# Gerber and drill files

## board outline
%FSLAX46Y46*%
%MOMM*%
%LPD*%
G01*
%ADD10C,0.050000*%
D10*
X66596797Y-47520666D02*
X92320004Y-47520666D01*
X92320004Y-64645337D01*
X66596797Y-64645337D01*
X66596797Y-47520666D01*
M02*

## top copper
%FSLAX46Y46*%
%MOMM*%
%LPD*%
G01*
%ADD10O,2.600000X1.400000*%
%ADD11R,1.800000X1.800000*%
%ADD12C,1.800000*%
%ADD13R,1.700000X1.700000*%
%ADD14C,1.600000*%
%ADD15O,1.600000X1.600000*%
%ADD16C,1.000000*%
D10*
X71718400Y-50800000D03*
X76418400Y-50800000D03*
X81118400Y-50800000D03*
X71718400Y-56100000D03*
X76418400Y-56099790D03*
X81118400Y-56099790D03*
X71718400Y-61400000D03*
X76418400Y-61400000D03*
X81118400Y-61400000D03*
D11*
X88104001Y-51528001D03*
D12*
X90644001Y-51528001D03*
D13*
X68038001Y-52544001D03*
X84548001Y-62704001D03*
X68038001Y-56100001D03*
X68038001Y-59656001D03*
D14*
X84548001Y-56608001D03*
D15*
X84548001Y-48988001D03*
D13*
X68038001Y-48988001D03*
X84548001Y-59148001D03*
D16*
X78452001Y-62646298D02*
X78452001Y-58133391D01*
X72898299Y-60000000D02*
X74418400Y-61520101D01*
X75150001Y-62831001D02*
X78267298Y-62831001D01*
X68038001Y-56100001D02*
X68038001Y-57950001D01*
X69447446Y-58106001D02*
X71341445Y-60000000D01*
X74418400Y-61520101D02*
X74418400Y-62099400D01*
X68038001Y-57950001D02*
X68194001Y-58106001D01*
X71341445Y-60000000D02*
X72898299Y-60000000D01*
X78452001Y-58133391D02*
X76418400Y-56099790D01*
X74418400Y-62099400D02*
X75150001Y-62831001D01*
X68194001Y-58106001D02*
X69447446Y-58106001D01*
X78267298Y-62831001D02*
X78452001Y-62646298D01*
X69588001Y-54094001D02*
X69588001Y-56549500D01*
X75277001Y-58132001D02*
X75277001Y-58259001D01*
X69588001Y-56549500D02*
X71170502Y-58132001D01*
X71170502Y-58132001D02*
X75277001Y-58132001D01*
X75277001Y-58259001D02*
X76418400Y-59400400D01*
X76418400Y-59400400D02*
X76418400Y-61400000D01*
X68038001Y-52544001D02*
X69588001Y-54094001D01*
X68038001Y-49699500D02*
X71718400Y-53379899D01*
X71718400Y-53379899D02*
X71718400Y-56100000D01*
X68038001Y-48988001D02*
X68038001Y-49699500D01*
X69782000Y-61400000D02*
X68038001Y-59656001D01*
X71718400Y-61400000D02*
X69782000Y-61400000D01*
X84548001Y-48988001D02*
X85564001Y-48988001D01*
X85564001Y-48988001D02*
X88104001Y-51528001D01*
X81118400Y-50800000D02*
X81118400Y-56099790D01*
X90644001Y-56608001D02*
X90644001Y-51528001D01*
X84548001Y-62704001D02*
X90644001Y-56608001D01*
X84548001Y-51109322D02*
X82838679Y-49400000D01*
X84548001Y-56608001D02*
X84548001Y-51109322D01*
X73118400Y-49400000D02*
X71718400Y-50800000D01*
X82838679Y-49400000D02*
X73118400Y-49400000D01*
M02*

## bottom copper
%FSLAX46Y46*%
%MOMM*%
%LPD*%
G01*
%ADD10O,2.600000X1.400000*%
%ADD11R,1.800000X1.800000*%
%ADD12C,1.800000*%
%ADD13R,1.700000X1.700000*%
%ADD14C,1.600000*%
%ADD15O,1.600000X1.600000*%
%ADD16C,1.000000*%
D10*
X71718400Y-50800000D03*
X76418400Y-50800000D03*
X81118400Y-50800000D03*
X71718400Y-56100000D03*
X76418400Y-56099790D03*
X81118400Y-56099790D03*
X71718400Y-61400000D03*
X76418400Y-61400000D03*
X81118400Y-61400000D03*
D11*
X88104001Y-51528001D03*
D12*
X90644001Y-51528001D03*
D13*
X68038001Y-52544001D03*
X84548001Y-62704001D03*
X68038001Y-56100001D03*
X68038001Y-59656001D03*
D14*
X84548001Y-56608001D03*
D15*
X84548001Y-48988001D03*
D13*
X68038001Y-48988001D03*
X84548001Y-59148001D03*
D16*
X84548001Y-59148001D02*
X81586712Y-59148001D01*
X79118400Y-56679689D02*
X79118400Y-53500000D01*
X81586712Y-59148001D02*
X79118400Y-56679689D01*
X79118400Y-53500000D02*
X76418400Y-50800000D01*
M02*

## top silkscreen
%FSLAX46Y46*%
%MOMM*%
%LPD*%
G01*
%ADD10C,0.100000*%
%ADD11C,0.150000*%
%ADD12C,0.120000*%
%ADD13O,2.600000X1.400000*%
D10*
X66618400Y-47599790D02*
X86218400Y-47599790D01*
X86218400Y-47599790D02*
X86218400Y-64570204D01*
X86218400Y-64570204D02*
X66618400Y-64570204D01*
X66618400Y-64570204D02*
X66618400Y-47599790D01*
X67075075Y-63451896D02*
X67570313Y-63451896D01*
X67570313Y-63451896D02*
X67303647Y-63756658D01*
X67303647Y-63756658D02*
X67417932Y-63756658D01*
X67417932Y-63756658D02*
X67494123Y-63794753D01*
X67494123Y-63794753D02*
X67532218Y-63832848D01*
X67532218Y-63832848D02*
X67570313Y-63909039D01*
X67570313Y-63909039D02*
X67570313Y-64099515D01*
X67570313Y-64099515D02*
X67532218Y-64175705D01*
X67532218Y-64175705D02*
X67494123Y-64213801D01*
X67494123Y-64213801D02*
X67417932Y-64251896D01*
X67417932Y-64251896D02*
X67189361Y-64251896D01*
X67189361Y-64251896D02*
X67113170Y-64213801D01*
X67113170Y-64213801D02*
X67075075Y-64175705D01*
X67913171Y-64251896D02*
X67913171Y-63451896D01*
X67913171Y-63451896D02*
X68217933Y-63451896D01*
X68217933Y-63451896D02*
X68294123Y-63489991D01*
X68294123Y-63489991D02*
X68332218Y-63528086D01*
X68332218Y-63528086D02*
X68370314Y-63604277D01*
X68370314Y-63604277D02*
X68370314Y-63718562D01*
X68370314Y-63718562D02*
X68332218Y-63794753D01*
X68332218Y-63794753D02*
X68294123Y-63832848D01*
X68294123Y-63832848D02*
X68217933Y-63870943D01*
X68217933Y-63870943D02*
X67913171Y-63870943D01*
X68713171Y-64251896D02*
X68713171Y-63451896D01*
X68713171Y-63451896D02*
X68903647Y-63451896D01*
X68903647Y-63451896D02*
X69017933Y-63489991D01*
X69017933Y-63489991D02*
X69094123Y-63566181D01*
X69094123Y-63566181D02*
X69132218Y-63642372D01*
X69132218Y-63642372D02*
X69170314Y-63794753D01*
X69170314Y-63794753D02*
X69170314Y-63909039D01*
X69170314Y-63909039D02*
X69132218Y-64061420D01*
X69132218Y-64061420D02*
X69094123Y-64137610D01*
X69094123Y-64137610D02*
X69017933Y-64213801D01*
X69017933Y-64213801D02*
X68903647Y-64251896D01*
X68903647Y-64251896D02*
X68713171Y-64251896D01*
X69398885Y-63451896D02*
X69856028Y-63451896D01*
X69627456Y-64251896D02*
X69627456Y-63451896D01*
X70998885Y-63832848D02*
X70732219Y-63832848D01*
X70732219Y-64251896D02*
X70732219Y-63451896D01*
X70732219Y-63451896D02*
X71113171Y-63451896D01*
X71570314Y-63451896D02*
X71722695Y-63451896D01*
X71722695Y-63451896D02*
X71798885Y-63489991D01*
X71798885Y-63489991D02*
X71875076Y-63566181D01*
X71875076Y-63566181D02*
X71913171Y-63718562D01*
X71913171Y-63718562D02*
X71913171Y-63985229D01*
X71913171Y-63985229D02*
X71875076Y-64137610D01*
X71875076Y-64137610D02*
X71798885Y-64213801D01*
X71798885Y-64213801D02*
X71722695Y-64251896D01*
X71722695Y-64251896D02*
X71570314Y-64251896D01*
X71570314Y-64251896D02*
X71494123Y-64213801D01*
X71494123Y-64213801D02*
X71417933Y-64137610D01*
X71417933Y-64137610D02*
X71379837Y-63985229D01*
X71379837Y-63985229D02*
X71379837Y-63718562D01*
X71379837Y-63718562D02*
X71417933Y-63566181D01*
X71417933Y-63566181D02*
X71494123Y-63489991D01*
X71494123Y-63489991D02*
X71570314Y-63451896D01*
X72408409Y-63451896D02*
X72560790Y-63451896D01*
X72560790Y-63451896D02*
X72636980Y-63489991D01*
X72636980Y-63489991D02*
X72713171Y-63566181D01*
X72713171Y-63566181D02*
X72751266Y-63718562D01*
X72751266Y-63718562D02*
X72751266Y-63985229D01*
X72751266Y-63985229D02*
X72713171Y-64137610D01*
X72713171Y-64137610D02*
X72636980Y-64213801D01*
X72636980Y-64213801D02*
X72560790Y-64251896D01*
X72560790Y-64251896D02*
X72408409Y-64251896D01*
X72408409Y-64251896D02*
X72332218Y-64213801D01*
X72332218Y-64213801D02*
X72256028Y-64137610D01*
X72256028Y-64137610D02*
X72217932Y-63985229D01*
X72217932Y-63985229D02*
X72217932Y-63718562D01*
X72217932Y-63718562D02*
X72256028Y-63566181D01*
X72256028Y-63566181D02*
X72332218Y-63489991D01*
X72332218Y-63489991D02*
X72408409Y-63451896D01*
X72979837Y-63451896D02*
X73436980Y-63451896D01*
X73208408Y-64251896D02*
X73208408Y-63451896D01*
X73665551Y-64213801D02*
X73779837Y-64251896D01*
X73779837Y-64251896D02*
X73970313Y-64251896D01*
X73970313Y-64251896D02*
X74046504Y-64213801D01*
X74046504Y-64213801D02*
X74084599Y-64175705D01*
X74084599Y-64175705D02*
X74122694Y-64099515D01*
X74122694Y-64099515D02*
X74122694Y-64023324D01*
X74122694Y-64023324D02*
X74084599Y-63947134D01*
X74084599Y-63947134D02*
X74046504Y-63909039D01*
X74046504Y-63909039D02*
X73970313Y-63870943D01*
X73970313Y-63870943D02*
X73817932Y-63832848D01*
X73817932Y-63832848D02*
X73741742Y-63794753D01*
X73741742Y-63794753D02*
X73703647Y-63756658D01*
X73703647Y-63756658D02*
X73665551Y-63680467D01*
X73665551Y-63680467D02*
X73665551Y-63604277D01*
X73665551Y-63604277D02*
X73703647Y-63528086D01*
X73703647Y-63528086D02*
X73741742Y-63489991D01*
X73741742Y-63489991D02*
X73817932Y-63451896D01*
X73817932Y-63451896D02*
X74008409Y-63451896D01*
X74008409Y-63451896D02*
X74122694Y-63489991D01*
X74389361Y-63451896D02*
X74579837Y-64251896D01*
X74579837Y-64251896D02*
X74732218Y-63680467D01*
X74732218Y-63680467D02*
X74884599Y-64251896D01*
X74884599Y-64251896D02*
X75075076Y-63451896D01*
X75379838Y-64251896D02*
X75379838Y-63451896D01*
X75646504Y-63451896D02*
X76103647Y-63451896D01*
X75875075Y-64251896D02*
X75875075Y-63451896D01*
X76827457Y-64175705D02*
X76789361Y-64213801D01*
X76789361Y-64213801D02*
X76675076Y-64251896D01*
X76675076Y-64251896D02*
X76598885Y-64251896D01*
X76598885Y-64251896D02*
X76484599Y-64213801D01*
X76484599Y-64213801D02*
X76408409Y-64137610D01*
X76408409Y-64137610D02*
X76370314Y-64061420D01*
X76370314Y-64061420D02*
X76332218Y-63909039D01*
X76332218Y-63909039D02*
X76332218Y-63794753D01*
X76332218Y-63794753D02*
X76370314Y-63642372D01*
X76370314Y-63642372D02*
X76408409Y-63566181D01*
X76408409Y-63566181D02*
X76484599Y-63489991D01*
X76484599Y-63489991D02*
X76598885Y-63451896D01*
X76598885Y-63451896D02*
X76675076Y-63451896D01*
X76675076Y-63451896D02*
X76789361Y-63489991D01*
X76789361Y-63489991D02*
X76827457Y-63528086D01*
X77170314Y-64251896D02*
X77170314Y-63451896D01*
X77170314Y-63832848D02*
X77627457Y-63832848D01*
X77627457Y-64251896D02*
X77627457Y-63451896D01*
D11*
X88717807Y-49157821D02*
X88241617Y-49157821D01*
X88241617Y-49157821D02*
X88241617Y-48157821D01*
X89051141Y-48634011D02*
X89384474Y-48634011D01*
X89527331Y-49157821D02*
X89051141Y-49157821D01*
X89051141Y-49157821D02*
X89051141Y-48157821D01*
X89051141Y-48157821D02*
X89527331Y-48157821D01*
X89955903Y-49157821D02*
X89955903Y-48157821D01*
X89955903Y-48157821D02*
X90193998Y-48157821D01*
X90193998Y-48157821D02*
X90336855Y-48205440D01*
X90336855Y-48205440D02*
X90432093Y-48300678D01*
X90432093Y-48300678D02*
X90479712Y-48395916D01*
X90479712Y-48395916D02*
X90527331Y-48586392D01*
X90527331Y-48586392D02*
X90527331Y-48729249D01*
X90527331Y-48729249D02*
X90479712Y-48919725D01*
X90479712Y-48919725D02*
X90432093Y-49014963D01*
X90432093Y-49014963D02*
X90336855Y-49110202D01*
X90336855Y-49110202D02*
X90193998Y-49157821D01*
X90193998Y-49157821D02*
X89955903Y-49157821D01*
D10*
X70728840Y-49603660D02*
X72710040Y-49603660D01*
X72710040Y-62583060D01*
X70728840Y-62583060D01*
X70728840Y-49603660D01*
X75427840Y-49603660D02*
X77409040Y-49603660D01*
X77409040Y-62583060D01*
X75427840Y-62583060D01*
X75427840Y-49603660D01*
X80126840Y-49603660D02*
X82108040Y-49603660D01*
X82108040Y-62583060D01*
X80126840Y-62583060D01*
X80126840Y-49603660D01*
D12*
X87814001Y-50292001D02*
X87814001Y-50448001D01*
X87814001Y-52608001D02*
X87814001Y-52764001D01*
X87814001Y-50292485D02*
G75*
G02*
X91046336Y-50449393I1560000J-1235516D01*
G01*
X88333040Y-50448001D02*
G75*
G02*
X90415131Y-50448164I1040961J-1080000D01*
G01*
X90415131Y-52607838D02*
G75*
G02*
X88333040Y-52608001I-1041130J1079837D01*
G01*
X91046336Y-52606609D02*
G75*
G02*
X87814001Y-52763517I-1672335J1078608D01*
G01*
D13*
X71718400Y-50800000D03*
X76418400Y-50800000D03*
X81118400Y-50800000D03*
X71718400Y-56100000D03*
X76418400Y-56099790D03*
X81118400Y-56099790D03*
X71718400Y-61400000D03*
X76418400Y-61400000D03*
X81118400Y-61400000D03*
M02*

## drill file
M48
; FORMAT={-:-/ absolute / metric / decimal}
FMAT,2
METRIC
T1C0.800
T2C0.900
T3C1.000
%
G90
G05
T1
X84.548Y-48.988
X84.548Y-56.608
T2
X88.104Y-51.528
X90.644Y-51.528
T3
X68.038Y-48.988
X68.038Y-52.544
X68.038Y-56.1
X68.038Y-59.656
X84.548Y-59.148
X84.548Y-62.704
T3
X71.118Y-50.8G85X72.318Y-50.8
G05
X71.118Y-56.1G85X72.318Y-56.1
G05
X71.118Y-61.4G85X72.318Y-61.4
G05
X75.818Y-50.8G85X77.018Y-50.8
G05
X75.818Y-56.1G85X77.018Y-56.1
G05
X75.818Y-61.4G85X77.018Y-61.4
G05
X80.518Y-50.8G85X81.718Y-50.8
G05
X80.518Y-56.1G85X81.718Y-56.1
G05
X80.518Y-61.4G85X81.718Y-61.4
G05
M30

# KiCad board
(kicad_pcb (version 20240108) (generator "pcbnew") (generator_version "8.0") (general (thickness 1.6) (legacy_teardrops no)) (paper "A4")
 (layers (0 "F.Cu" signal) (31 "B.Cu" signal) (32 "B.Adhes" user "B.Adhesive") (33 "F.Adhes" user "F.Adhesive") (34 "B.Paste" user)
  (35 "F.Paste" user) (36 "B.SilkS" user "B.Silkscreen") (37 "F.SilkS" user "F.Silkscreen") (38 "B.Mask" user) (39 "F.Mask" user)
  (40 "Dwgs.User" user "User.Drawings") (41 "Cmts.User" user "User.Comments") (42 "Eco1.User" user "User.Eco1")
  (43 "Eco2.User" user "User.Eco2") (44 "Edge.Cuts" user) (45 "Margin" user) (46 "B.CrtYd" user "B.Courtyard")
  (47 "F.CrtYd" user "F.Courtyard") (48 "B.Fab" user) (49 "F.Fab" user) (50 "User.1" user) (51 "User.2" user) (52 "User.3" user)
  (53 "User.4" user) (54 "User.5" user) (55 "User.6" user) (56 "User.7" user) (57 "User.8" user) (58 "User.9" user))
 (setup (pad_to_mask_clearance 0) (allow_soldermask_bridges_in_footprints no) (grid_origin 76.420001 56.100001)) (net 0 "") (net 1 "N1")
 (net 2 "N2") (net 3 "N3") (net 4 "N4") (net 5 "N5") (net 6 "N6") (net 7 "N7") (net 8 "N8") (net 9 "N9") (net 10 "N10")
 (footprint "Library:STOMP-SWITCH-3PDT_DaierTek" (layer "F.Cu") (at 76.41844 55.59806)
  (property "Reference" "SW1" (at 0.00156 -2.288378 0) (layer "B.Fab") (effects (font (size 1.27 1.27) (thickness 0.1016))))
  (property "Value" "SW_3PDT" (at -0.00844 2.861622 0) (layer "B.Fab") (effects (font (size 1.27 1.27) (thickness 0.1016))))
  (fp_rect (start -5.6896 -5.9944) (end -3.7084 6.985) (stroke (width 0.1) (type default)) (fill none) (layer "F.SilkS"))
  (fp_rect (start -0.9906 -5.9944) (end 0.9906 6.985) (stroke (width 0.1) (type default)) (fill none) (layer "F.SilkS"))
  (fp_rect (start 3.7084 -5.9944) (end 5.6896 6.985) (stroke (width 0.1) (type default)) (fill none) (layer "F.SilkS"))
  (pad "1" thru_hole oval (at -4.70004 -4.79806) (size 2.6 1.4) (drill oval 2.2 1) (layers "*.Cu" "F.Paste" "F.SilkS" "F.Mask")
   (remove_unused_layers no) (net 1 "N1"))
  (pad "2" thru_hole oval (at -0.00004 -4.79806) (size 2.6 1.4) (drill oval 2.2 1) (layers "*.Cu" "F.Paste" "F.SilkS" "F.Mask")
   (remove_unused_layers no) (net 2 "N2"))
  (pad "3" thru_hole oval (at 4.69996 -4.79806) (size 2.6 1.4) (drill oval 2.2 1) (layers "*.Cu" "F.Paste" "F.SilkS" "F.Mask")
   (remove_unused_layers no) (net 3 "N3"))
  (pad "4" thru_hole oval (at -4.70004 0.50194) (size 2.6 1.4) (drill oval 2.2 1) (layers "*.Cu" "F.Paste" "F.SilkS" "F.Mask")
   (remove_unused_layers no) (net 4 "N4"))
  (pad "5" thru_hole oval (at -0.00004 0.50173) (size 2.6 1.4) (drill oval 2.2 1) (layers "*.Cu" "F.Paste" "F.SilkS" "F.Mask")
   (remove_unused_layers no) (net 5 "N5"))
  (pad "6" thru_hole oval (at 4.69996 0.50173) (size 2.6 1.4) (drill oval 2.2 1) (layers "*.Cu" "F.Paste" "F.SilkS" "F.Mask")
   (remove_unused_layers no) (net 3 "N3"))
  (pad "7" thru_hole oval (at -4.70004 5.80194) (size 2.6 1.4) (drill oval 2.2 1) (layers "*.Cu" "F.Paste" "F.SilkS" "F.Mask")
   (remove_unused_layers no) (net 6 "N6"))
  (pad "8" thru_hole oval (at -0.00004 5.80194) (size 2.6 1.4) (drill oval 2.2 1) (layers "*.Cu" "F.Paste" "F.SilkS" "F.Mask")
   (remove_unused_layers no) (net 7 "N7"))
  (pad "9" thru_hole oval (at 4.69996 5.80194) (size 2.6 1.4) (drill oval 2.2 1) (layers "*.Cu" "F.Paste" "F.SilkS" "F.Mask")
   (remove_unused_layers no) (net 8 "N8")))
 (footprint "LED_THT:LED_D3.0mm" (layer "F.Cu") (at 88.104001 51.528001)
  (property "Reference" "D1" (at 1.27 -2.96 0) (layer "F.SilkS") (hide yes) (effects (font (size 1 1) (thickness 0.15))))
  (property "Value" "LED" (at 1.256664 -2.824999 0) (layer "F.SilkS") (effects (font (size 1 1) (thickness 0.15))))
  (fp_line (start -0.29 -1.236) (end -0.29 -1.08) (stroke (width 0.12) (type solid)) (layer "F.SilkS"))
  (fp_line (start -0.29 1.08) (end -0.29 1.236) (stroke (width 0.12) (type solid)) (layer "F.SilkS"))
  (fp_arc (start -0.29 -1.235516) (mid 1.366487 -1.987659) (end 2.942335 -1.078608) (stroke (width 0.12) (type solid)) (layer "F.SilkS"))
  (fp_arc (start 0.229039 -1.08) (mid 1.270117 -1.5) (end 2.31113 -1.079837) (stroke (width 0.12) (type solid)) (layer "F.SilkS"))
  (fp_arc (start 2.31113 1.079837) (mid 1.270117 1.5) (end 0.229039 1.08) (stroke (width 0.12) (type solid)) (layer "F.SilkS"))
  (fp_arc (start 2.942335 1.078608) (mid 1.366487 1.987659) (end -0.29 1.235516) (stroke (width 0.12) (type solid)) (layer "F.SilkS"))
  (pad "1" thru_hole rect (at 0 0) (size 1.8 1.8) (drill 0.9) (layers "*.Cu" "*.Mask") (remove_unused_layers no) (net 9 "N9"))
  (pad "2" thru_hole circle (at 2.54 0) (size 1.8 1.8) (drill 0.9) (layers "*.Cu" "*.Mask") (remove_unused_layers no) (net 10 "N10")))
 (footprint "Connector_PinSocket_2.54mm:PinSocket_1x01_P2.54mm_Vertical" (layer "B.Cu") (at 68.038001 52.544001 180)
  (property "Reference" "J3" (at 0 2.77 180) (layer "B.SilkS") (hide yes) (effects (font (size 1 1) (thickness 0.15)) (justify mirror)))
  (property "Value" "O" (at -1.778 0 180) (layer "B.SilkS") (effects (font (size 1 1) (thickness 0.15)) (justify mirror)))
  (pad "1" thru_hole rect (at 0 0 180) (size 1.7 1.7) (drill 1) (layers "*.Cu" "*.Mask") (remove_unused_layers no) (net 7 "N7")))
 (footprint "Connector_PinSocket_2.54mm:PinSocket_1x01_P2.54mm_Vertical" (layer "B.Cu") (at 84.548001 62.704001 180)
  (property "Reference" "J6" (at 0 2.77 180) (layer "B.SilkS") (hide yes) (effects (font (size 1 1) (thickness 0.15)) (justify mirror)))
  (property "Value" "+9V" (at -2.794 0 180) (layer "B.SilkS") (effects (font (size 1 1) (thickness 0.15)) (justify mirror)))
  (pad "1" thru_hole rect (at 0 0 180) (size 1.7 1.7) (drill 1) (layers "*.Cu" "*.Mask") (remove_unused_layers no) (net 10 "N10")))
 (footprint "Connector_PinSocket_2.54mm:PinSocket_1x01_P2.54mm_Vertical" (layer "B.Cu") (at 68.038001 56.100001 180)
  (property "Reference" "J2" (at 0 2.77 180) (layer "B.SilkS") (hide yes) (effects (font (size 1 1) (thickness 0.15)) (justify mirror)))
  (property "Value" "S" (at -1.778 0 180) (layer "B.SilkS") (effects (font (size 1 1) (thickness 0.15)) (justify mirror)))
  (pad "1" thru_hole rect (at 0 0 180) (size 1.7 1.7) (drill 1) (layers "*.Cu" "*.Mask") (remove_unused_layers no) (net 5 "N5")))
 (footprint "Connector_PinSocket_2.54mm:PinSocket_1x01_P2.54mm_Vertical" (layer "B.Cu") (at 68.038001 59.656001 180)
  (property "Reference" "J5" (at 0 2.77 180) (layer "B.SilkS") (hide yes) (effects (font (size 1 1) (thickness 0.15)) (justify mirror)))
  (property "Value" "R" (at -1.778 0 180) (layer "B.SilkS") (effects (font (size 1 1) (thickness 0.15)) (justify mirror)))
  (pad "1" thru_hole rect (at 0 0 180) (size 1.7 1.7) (drill 1) (layers "*.Cu" "*.Mask") (remove_unused_layers no) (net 6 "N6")))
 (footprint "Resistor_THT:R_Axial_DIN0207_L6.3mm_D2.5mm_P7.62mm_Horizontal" (layer "B.Cu") (at 84.548001 56.608001 90)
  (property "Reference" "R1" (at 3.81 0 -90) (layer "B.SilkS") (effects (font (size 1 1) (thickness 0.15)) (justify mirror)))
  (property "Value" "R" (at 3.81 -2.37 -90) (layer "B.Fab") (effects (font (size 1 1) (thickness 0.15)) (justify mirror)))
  (pad "1" thru_hole circle (at 0 0 90) (size 1.6 1.6) (drill 0.8) (layers "*.Cu" "*.Mask") (remove_unused_layers no) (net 1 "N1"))
  (pad "2" thru_hole oval (at 7.62 0 90) (size 1.6 1.6) (drill 0.8) (layers "*.Cu" "*.Mask") (remove_unused_layers no) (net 9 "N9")))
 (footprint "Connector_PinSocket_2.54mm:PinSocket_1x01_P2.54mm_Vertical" (layer "B.Cu") (at 68.038001 48.988001 180)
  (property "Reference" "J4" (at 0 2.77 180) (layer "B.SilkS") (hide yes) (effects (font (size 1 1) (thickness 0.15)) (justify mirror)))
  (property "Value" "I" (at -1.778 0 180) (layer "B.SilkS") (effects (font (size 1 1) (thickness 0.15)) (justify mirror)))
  (pad "1" thru_hole rect (at 0 0 180) (size 1.7 1.7) (drill 1) (layers "*.Cu" "*.Mask") (remove_unused_layers no) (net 4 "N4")))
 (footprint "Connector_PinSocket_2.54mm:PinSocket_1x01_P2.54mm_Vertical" (layer "B.Cu") (at 84.548001 59.148001 180)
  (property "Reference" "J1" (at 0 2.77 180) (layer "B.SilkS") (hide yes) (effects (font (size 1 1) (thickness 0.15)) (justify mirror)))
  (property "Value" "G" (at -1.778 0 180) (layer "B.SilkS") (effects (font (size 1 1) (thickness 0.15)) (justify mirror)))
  (pad "1" thru_hole rect (at 0 0 180) (size 1.7 1.7) (drill 1) (layers "*.Cu" "*.Mask") (remove_unused_layers no) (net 2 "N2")))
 (gr_line (start 66.6184 47.59979) (end 86.2184 47.59979) (stroke (width 0.1) (type default)) (layer "F.SilkS"))
 (gr_line (start 86.2184 47.59979) (end 86.2184 64.570204) (stroke (width 0.1) (type default)) (layer "F.SilkS"))
 (gr_line (start 86.2184 64.570204) (end 66.6184 64.570204) (stroke (width 0.1) (type default)) (layer "F.SilkS"))
 (gr_line (start 66.6184 64.570204) (end 66.6184 47.59979) (stroke (width 0.1) (type default)) (layer "F.SilkS"))
 (gr_rect (start 66.596797 47.520666) (end 92.320004 64.645337) (stroke (width 0.05) (type default)) (fill none) (layer "Edge.Cuts"))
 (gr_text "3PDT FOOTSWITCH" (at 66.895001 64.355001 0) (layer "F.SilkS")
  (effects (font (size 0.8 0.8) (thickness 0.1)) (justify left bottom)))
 (segment (start 84.548001 59.148001) (end 81.586712 59.148001) (width 1) (layer "B.Cu") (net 2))
 (segment (start 79.1184 56.679689) (end 79.1184 53.5) (width 1) (layer "B.Cu") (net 2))
 (segment (start 81.586712 59.148001) (end 79.1184 56.679689) (width 1) (layer "B.Cu") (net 2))
 (segment (start 79.1184 53.5) (end 76.4184 50.8) (width 1) (layer "B.Cu") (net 2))
 (segment (start 78.452001 62.646298) (end 78.452001 58.133391) (width 1) (layer "F.Cu") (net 5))
 (segment (start 72.898299 60) (end 74.4184 61.520101) (width 1) (layer "F.Cu") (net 5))
 (segment (start 75.150001 62.831001) (end 78.267298 62.831001) (width 1) (layer "F.Cu") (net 5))
 (segment (start 68.038001 56.100001) (end 68.038001 57.950001) (width 1) (layer "F.Cu") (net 5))
 (segment (start 69.447446 58.106001) (end 71.341445 60) (width 1) (layer "F.Cu") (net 5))
 (segment (start 74.4184 61.520101) (end 74.4184 62.0994) (width 1) (layer "F.Cu") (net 5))
 (segment (start 68.038001 57.950001) (end 68.194001 58.106001) (width 1) (layer "F.Cu") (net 5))
 (segment (start 71.341445 60) (end 72.898299 60) (width 1) (layer "F.Cu") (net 5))
 (segment (start 78.452001 58.133391) (end 76.4184 56.09979) (width 1) (layer "F.Cu") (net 5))
 (segment (start 74.4184 62.0994) (end 75.150001 62.831001) (width 1) (layer "F.Cu") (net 5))
 (segment (start 68.194001 58.106001) (end 69.447446 58.106001) (width 1) (layer "F.Cu") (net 5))
 (segment (start 78.267298 62.831001) (end 78.452001 62.646298) (width 1) (layer "F.Cu") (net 5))
 (segment (start 69.588001 54.094001) (end 69.588001 56.5495) (width 1) (layer "F.Cu") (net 7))
 (segment (start 75.277001 58.132001) (end 75.277001 58.259001) (width 1) (layer "F.Cu") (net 7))
 (segment (start 69.588001 56.5495) (end 71.170502 58.132001) (width 1) (layer "F.Cu") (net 7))
 (segment (start 71.170502 58.132001) (end 75.277001 58.132001) (width 1) (layer "F.Cu") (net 7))
 (segment (start 75.277001 58.259001) (end 76.4184 59.4004) (width 1) (layer "F.Cu") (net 7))
 (segment (start 76.4184 59.4004) (end 76.4184 61.4) (width 1) (layer "F.Cu") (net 7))
 (segment (start 68.038001 52.544001) (end 69.588001 54.094001) (width 1) (layer "F.Cu") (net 7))
 (segment (start 68.038001 49.6995) (end 71.7184 53.379899) (width 1) (layer "F.Cu") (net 4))
 (segment (start 71.7184 53.379899) (end 71.7184 56.1) (width 1) (layer "F.Cu") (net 4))
 (segment (start 68.038001 48.988001) (end 68.038001 49.6995) (width 1) (layer "F.Cu") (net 4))
 (segment (start 69.782 61.4) (end 68.038001 59.656001) (width 1) (layer "F.Cu") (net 6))
 (segment (start 71.7184 61.4) (end 69.782 61.4) (width 1) (layer "F.Cu") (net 6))
 (segment (start 84.548001 48.988001) (end 85.564001 48.988001) (width 1) (layer "F.Cu") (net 9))
 (segment (start 85.564001 48.988001) (end 88.104001 51.528001) (width 1) (layer "F.Cu") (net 9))
 (segment (start 81.1184 50.8) (end 81.1184 56.09979) (width 1) (layer "F.Cu") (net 3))
 (segment (start 90.644001 56.608001) (end 90.644001 51.528001) (width 1) (layer "F.Cu") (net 10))
 (segment (start 84.548001 62.704001) (end 90.644001 56.608001) (width 1) (layer "F.Cu") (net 10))
 (segment (start 84.548001 51.109322) (end 82.838679 49.4) (width 1) (layer "F.Cu") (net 1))
 (segment (start 84.548001 56.608001) (end 84.548001 51.109322) (width 1) (layer "F.Cu") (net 1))
 (segment (start 73.1184 49.4) (end 71.7184 50.8) (width 1) (layer "F.Cu") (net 1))
 (segment (start 82.838679 49.4) (end 73.1184 49.4) (width 1) (layer "F.Cu") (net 1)))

